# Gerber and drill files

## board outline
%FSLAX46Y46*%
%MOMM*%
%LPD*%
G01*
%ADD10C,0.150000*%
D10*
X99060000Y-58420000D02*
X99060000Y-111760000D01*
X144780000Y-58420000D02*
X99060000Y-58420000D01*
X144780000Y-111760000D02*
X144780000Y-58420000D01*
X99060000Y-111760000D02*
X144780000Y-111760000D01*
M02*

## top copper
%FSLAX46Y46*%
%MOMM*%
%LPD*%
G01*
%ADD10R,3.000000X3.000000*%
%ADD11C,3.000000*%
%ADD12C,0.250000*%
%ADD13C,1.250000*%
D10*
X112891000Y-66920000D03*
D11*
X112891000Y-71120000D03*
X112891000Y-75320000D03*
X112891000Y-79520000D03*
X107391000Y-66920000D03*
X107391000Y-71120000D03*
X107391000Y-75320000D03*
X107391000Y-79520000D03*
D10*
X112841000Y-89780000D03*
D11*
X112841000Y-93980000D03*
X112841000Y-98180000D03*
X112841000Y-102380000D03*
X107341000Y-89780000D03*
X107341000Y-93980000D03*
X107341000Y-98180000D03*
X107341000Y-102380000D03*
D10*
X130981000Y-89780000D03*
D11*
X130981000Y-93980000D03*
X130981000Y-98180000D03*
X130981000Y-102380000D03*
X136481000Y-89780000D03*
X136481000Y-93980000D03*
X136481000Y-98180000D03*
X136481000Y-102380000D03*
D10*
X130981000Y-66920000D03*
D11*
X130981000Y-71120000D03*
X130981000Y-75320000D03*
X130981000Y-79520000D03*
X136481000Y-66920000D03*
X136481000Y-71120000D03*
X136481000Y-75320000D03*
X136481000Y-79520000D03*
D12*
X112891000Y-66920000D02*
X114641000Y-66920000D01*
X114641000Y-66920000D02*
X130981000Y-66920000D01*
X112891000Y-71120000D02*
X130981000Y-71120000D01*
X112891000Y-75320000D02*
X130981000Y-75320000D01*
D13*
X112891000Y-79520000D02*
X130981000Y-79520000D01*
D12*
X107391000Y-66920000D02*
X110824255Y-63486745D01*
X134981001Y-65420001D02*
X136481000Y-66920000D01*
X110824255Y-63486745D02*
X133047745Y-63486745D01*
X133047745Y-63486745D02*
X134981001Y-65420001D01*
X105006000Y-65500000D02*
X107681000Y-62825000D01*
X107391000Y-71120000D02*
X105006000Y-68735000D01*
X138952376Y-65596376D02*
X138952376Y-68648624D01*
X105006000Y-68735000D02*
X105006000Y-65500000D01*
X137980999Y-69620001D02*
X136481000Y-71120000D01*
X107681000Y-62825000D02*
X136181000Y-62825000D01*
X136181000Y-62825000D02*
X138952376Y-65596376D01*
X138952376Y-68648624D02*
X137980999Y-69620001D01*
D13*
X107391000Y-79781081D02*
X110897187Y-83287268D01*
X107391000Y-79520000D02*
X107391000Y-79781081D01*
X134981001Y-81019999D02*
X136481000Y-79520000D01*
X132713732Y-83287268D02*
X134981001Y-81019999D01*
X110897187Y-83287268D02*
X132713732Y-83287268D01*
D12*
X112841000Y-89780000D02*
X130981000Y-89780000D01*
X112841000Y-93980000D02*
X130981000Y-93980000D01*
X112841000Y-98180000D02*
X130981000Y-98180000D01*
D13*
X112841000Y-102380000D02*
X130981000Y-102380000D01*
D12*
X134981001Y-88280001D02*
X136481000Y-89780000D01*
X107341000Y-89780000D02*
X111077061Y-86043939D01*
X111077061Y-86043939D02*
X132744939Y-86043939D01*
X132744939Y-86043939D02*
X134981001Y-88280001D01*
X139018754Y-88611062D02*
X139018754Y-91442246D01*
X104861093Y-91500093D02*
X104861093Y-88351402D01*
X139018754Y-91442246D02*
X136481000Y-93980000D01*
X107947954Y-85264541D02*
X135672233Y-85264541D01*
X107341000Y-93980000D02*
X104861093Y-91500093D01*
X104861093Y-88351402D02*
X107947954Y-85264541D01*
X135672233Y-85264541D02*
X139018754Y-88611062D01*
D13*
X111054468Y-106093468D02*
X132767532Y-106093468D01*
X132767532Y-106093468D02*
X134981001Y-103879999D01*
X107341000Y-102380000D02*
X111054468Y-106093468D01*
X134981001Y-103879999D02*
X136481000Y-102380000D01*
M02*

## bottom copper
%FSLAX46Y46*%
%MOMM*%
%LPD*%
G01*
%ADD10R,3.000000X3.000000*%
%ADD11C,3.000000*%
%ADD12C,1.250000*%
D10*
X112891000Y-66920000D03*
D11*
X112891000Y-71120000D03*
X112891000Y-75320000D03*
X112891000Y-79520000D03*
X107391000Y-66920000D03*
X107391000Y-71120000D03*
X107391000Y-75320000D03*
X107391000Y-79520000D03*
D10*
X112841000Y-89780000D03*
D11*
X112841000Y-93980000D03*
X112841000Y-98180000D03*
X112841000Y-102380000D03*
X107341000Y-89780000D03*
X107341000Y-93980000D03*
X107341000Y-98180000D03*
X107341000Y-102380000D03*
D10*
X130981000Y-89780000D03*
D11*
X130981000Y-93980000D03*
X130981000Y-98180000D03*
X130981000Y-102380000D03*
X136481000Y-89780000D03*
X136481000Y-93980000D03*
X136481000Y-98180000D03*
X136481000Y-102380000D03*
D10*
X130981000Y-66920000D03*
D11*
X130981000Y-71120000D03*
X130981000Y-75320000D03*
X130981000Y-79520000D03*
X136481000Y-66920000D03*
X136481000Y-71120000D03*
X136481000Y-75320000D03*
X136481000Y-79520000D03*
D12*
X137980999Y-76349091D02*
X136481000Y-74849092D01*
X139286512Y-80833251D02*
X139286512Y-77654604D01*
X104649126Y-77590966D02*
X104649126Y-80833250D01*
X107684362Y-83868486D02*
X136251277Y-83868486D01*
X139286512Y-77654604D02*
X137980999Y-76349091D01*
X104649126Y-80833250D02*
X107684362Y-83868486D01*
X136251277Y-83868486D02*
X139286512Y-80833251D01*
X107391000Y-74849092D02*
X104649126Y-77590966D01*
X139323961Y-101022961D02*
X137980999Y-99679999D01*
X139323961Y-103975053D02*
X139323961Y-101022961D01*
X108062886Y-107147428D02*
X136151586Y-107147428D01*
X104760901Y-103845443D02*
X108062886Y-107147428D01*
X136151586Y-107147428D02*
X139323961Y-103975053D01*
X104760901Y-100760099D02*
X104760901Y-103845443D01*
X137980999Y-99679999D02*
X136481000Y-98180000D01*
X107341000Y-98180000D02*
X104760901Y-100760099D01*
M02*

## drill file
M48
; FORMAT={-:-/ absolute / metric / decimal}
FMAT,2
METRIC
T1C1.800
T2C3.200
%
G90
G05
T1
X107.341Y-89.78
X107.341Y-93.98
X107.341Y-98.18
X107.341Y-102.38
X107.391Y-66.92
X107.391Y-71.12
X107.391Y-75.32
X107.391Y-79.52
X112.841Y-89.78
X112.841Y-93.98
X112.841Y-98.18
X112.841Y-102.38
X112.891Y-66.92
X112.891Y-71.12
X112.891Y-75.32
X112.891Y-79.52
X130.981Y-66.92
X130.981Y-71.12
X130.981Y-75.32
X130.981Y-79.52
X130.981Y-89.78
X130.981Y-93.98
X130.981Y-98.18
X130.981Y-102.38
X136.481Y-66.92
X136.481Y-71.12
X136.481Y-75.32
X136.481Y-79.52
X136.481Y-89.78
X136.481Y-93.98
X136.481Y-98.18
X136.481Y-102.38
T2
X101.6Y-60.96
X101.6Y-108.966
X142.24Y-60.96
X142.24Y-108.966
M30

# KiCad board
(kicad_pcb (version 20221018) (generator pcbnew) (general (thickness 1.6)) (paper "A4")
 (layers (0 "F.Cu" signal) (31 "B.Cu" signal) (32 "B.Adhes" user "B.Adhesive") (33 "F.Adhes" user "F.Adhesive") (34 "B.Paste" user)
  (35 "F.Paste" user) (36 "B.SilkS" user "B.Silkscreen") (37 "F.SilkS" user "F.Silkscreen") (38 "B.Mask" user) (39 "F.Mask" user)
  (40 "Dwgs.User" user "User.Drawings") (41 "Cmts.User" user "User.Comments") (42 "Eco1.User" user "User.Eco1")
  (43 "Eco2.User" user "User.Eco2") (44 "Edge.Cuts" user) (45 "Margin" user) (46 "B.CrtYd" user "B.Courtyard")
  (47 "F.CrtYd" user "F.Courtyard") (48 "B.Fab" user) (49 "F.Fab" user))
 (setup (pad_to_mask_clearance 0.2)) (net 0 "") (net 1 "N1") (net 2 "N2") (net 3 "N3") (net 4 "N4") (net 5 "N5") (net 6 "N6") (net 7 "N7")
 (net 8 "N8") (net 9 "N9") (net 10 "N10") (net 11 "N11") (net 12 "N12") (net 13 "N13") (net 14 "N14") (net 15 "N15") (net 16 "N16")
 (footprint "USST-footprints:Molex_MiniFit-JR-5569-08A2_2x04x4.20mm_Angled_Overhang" (layer "F.Cu") (at 112.891 66.92 -90)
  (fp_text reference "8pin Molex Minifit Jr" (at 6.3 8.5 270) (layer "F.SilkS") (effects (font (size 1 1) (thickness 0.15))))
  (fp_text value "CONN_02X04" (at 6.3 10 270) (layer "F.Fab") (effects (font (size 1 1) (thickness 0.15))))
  (pad "1" thru_hole rect (at 0 0 270) (size 3 3) (drill 1.8) (layers "*.Cu" "*.Mask") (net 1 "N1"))
  (pad "2" thru_hole circle (at 4.2 0 270) (size 3 3) (drill 1.8) (layers "*.Cu" "*.Mask") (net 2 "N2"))
  (pad "3" thru_hole circle (at 8.4 0 270) (size 3 3) (drill 1.8) (layers "*.Cu" "*.Mask") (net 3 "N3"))
  (pad "4" thru_hole circle (at 12.6 0 270) (size 3 3) (drill 1.8) (layers "*.Cu" "*.Mask") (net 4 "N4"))
  (pad "5" thru_hole circle (at 0 5.5 270) (size 3 3) (drill 1.8) (layers "*.Cu" "*.Mask") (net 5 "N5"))
  (pad "6" thru_hole circle (at 4.2 5.5 270) (size 3 3) (drill 1.8) (layers "*.Cu" "*.Mask") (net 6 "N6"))
  (pad "7" thru_hole circle (at 8.4 5.5 270) (size 3 3) (drill 1.8) (layers "*.Cu" "*.Mask") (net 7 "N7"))
  (pad "8" thru_hole circle (at 12.6 5.5 270) (size 3 3) (drill 1.8) (layers "*.Cu" "*.Mask") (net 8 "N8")))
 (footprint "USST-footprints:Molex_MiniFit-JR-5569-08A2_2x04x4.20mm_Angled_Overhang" (layer "F.Cu") (at 112.841 89.78 -90)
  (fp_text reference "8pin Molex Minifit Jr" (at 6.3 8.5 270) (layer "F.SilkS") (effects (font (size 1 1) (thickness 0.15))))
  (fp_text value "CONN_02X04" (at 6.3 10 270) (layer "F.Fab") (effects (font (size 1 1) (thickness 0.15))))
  (pad "1" thru_hole rect (at 0 0 270) (size 3 3) (drill 1.8) (layers "*.Cu" "*.Mask") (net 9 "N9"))
  (pad "2" thru_hole circle (at 4.2 0 270) (size 3 3) (drill 1.8) (layers "*.Cu" "*.Mask") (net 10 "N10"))
  (pad "3" thru_hole circle (at 8.4 0 270) (size 3 3) (drill 1.8) (layers "*.Cu" "*.Mask") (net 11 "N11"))
  (pad "4" thru_hole circle (at 12.6 0 270) (size 3 3) (drill 1.8) (layers "*.Cu" "*.Mask") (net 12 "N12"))
  (pad "5" thru_hole circle (at 0 5.5 270) (size 3 3) (drill 1.8) (layers "*.Cu" "*.Mask") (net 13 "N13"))
  (pad "6" thru_hole circle (at 4.2 5.5 270) (size 3 3) (drill 1.8) (layers "*.Cu" "*.Mask") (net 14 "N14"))
  (pad "7" thru_hole circle (at 8.4 5.5 270) (size 3 3) (drill 1.8) (layers "*.Cu" "*.Mask") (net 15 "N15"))
  (pad "8" thru_hole circle (at 12.6 5.5 270) (size 3 3) (drill 1.8) (layers "*.Cu" "*.Mask") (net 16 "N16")))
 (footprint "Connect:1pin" (layer "F.Cu") (at 142.24 60.96)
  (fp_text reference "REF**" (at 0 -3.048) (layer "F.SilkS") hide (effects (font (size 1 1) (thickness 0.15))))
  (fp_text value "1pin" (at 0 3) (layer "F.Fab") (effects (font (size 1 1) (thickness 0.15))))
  (pad "" np_thru_hole circle (at 0 0) (size 3.2 3.2) (drill 3.2) (layers "*.Cu" "*.Mask")))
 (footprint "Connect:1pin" (layer "F.Cu") (at 101.6 60.96)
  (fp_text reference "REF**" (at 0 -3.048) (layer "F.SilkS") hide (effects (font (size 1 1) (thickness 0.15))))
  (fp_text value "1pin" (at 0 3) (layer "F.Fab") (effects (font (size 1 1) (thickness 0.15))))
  (pad "" np_thru_hole circle (at 0 0) (size 3.2 3.2) (drill 3.2) (layers "*.Cu" "*.Mask")))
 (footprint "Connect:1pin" (layer "F.Cu") (at 101.6 108.966)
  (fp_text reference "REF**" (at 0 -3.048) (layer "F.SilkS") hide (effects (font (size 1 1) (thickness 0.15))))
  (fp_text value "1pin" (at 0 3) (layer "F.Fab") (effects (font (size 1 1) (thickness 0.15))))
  (pad "" np_thru_hole circle (at 0 0) (size 3.2 3.2) (drill 3.2) (layers "*.Cu" "*.Mask")))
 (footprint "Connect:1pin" (layer "F.Cu") (at 142.24 108.966)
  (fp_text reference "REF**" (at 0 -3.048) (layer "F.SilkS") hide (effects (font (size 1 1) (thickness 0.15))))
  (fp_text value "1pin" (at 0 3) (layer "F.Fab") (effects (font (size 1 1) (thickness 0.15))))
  (pad "" np_thru_hole circle (at 0 0) (size 3.2 3.2) (drill 3.2) (layers "*.Cu" "*.Mask")))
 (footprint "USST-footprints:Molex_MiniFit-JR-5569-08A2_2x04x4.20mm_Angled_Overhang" (layer "B.Cu") (at 130.981 89.78 -90)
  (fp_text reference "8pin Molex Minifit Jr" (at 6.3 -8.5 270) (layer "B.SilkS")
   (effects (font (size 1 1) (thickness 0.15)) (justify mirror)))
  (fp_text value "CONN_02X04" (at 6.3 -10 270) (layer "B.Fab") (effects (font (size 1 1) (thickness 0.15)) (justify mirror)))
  (pad "1" thru_hole rect (at 0 0 270) (size 3 3) (drill 1.8) (layers "*.Cu" "*.Mask") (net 9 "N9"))
  (pad "2" thru_hole circle (at 4.2 0 270) (size 3 3) (drill 1.8) (layers "*.Cu" "*.Mask") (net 10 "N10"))
  (pad "3" thru_hole circle (at 8.4 0 270) (size 3 3) (drill 1.8) (layers "*.Cu" "*.Mask") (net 11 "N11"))
  (pad "4" thru_hole circle (at 12.6 0 270) (size 3 3) (drill 1.8) (layers "*.Cu" "*.Mask") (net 12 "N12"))
  (pad "5" thru_hole circle (at 0 -5.5 270) (size 3 3) (drill 1.8) (layers "*.Cu" "*.Mask") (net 13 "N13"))
  (pad "6" thru_hole circle (at 4.2 -5.5 270) (size 3 3) (drill 1.8) (layers "*.Cu" "*.Mask") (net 14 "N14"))
  (pad "7" thru_hole circle (at 8.4 -5.5 270) (size 3 3) (drill 1.8) (layers "*.Cu" "*.Mask") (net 15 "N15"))
  (pad "8" thru_hole circle (at 12.6 -5.5 270) (size 3 3) (drill 1.8) (layers "*.Cu" "*.Mask") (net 16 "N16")))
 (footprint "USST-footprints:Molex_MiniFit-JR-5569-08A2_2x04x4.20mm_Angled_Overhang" (layer "B.Cu") (at 130.981 66.92 -90)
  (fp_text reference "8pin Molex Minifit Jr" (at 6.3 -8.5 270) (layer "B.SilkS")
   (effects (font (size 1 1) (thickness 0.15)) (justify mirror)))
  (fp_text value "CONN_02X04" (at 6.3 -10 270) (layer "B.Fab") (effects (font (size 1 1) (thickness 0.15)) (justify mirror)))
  (pad "1" thru_hole rect (at 0 0 270) (size 3 3) (drill 1.8) (layers "*.Cu" "*.Mask") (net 1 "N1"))
  (pad "2" thru_hole circle (at 4.2 0 270) (size 3 3) (drill 1.8) (layers "*.Cu" "*.Mask") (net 2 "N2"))
  (pad "3" thru_hole circle (at 8.4 0 270) (size 3 3) (drill 1.8) (layers "*.Cu" "*.Mask") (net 3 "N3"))
  (pad "4" thru_hole circle (at 12.6 0 270) (size 3 3) (drill 1.8) (layers "*.Cu" "*.Mask") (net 4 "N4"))
  (pad "5" thru_hole circle (at 0 -5.5 270) (size 3 3) (drill 1.8) (layers "*.Cu" "*.Mask") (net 5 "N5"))
  (pad "6" thru_hole circle (at 4.2 -5.5 270) (size 3 3) (drill 1.8) (layers "*.Cu" "*.Mask") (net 6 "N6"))
  (pad "7" thru_hole circle (at 8.4 -5.5 270) (size 3 3) (drill 1.8) (layers "*.Cu" "*.Mask") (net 7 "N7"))
  (pad "8" thru_hole circle (at 12.6 -5.5 270) (size 3 3) (drill 1.8) (layers "*.Cu" "*.Mask") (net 8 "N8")))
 (gr_line (start 99.06 58.42) (end 99.06 111.76) (stroke (width 0.15) (type solid)) (layer "Edge.Cuts"))
 (gr_line (start 144.78 58.42) (end 99.06 58.42) (stroke (width 0.15) (type solid)) (layer "Edge.Cuts"))
 (gr_line (start 144.78 111.76) (end 144.78 58.42) (stroke (width 0.15) (type solid)) (layer "Edge.Cuts"))
 (gr_line (start 99.06 111.76) (end 144.78 111.76) (stroke (width 0.15) (type solid)) (layer "Edge.Cuts"))
 (segment (start 112.891 66.92) (end 114.641 66.92) (width 0.25) (layer "F.Cu") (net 1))
 (segment (start 114.641 66.92) (end 130.981 66.92) (width 0.25) (layer "F.Cu") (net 1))
 (segment (start 112.891 71.12) (end 130.981 71.12) (width 0.25) (layer "F.Cu") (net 2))
 (segment (start 112.891 75.32) (end 130.981 75.32) (width 0.25) (layer "F.Cu") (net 3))
 (segment (start 112.891 79.52) (end 130.981 79.52) (width 1.25) (layer "F.Cu") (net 4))
 (segment (start 107.391 66.92) (end 110.824255 63.486745) (width 0.25) (layer "F.Cu") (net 5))
 (segment (start 134.981001 65.420001) (end 136.481 66.92) (width 0.25) (layer "F.Cu") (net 5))
 (segment (start 110.824255 63.486745) (end 133.047745 63.486745) (width 0.25) (layer "F.Cu") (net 5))
 (segment (start 133.047745 63.486745) (end 134.981001 65.420001) (width 0.25) (layer "F.Cu") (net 5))
 (segment (start 105.006 65.5) (end 107.681 62.825) (width 0.25) (layer "F.Cu") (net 6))
 (segment (start 107.391 71.12) (end 105.006 68.735) (width 0.25) (layer "F.Cu") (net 6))
 (segment (start 138.952376 65.596376) (end 138.952376 68.648624) (width 0.25) (layer "F.Cu") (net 6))
 (segment (start 105.006 68.735) (end 105.006 65.5) (width 0.25) (layer "F.Cu") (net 6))
 (segment (start 137.980999 69.620001) (end 136.481 71.12) (width 0.25) (layer "F.Cu") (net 6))
 (segment (start 107.681 62.825) (end 136.181 62.825) (width 0.25) (layer "F.Cu") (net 6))
 (segment (start 136.181 62.825) (end 138.952376 65.596376) (width 0.25) (layer "F.Cu") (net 6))
 (segment (start 138.952376 68.648624) (end 137.980999 69.620001) (width 0.25) (layer "F.Cu") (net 6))
 (segment (start 137.980999 76.349091) (end 136.481 74.849092) (width 1.25) (layer "B.Cu") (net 7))
 (segment (start 139.286512 80.833251) (end 139.286512 77.654604) (width 1.25) (layer "B.Cu") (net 7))
 (segment (start 104.649126 77.590966) (end 104.649126 80.83325) (width 1.25) (layer "B.Cu") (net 7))
 (segment (start 107.684362 83.868486) (end 136.251277 83.868486) (width 1.25) (layer "B.Cu") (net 7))
 (segment (start 139.286512 77.654604) (end 137.980999 76.349091) (width 1.25) (layer "B.Cu") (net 7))
 (segment (start 104.649126 80.83325) (end 107.684362 83.868486) (width 1.25) (layer "B.Cu") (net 7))
 (segment (start 136.251277 83.868486) (end 139.286512 80.833251) (width 1.25) (layer "B.Cu") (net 7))
 (segment (start 107.391 74.849092) (end 104.649126 77.590966) (width 1.25) (layer "B.Cu") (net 7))
 (segment (start 107.391 79.781081) (end 110.897187 83.287268) (width 1.25) (layer "F.Cu") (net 8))
 (segment (start 107.391 79.52) (end 107.391 79.781081) (width 1.25) (layer "F.Cu") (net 8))
 (segment (start 134.981001 81.019999) (end 136.481 79.52) (width 1.25) (layer "F.Cu") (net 8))
 (segment (start 132.713732 83.287268) (end 134.981001 81.019999) (width 1.25) (layer "F.Cu") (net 8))
 (segment (start 110.897187 83.287268) (end 132.713732 83.287268) (width 1.25) (layer "F.Cu") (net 8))
 (segment (start 112.841 89.78) (end 130.981 89.78) (width 0.25) (layer "F.Cu") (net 9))
 (segment (start 112.841 93.98) (end 130.981 93.98) (width 0.25) (layer "F.Cu") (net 10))
 (segment (start 112.841 98.18) (end 130.981 98.18) (width 0.25) (layer "F.Cu") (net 11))
 (segment (start 112.841 102.38) (end 130.981 102.38) (width 1.25) (layer "F.Cu") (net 12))
 (segment (start 134.981001 88.280001) (end 136.481 89.78) (width 0.25) (layer "F.Cu") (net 13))
 (segment (start 107.341 89.78) (end 111.077061 86.043939) (width 0.25) (layer "F.Cu") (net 13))
 (segment (start 111.077061 86.043939) (end 132.744939 86.043939) (width 0.25) (layer "F.Cu") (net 13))
 (segment (start 132.744939 86.043939) (end 134.981001 88.280001) (width 0.25) (layer "F.Cu") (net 13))
 (segment (start 139.018754 88.611062) (end 139.018754 91.442246) (width 0.25) (layer "F.Cu") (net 14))
 (segment (start 104.861093 91.500093) (end 104.861093 88.351402) (width 0.25) (layer "F.Cu") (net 14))
 (segment (start 139.018754 91.442246) (end 136.481 93.98) (width 0.25) (layer "F.Cu") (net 14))
 (segment (start 107.947954 85.264541) (end 135.672233 85.264541) (width 0.25) (layer "F.Cu") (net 14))
 (segment (start 107.341 93.98) (end 104.861093 91.500093) (width 0.25) (layer "F.Cu") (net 14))
 (segment (start 104.861093 88.351402) (end 107.947954 85.264541) (width 0.25) (layer "F.Cu") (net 14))
 (segment (start 135.672233 85.264541) (end 139.018754 88.611062) (width 0.25) (layer "F.Cu") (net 14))
 (segment (start 139.323961 101.022961) (end 137.980999 99.679999) (width 1.25) (layer "B.Cu") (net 15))
 (segment (start 139.323961 103.975053) (end 139.323961 101.022961) (width 1.25) (layer "B.Cu") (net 15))
 (segment (start 108.062886 107.147428) (end 136.151586 107.147428) (width 1.25) (layer "B.Cu") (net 15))
 (segment (start 104.760901 103.845443) (end 108.062886 107.147428) (width 1.25) (layer "B.Cu") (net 15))
 (segment (start 136.151586 107.147428) (end 139.323961 103.975053) (width 1.25) (layer "B.Cu") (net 15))
 (segment (start 104.760901 100.760099) (end 104.760901 103.845443) (width 1.25) (layer "B.Cu") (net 15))
 (segment (start 137.980999 99.679999) (end 136.481 98.18) (width 1.25) (layer "B.Cu") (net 15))
 (segment (start 107.341 98.18) (end 104.760901 100.760099) (width 1.25) (layer "B.Cu") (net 15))
 (segment (start 111.054468 106.093468) (end 132.767532 106.093468) (width 1.25) (layer "F.Cu") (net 16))
 (segment (start 132.767532 106.093468) (end 134.981001 103.879999) (width 1.25) (layer "F.Cu") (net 16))
 (segment (start 107.341 102.38) (end 111.054468 106.093468) (width 1.25) (layer "F.Cu") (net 16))
 (segment (start 134.981001 103.879999) (end 136.481 102.38) (width 1.25) (layer "F.Cu") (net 16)))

